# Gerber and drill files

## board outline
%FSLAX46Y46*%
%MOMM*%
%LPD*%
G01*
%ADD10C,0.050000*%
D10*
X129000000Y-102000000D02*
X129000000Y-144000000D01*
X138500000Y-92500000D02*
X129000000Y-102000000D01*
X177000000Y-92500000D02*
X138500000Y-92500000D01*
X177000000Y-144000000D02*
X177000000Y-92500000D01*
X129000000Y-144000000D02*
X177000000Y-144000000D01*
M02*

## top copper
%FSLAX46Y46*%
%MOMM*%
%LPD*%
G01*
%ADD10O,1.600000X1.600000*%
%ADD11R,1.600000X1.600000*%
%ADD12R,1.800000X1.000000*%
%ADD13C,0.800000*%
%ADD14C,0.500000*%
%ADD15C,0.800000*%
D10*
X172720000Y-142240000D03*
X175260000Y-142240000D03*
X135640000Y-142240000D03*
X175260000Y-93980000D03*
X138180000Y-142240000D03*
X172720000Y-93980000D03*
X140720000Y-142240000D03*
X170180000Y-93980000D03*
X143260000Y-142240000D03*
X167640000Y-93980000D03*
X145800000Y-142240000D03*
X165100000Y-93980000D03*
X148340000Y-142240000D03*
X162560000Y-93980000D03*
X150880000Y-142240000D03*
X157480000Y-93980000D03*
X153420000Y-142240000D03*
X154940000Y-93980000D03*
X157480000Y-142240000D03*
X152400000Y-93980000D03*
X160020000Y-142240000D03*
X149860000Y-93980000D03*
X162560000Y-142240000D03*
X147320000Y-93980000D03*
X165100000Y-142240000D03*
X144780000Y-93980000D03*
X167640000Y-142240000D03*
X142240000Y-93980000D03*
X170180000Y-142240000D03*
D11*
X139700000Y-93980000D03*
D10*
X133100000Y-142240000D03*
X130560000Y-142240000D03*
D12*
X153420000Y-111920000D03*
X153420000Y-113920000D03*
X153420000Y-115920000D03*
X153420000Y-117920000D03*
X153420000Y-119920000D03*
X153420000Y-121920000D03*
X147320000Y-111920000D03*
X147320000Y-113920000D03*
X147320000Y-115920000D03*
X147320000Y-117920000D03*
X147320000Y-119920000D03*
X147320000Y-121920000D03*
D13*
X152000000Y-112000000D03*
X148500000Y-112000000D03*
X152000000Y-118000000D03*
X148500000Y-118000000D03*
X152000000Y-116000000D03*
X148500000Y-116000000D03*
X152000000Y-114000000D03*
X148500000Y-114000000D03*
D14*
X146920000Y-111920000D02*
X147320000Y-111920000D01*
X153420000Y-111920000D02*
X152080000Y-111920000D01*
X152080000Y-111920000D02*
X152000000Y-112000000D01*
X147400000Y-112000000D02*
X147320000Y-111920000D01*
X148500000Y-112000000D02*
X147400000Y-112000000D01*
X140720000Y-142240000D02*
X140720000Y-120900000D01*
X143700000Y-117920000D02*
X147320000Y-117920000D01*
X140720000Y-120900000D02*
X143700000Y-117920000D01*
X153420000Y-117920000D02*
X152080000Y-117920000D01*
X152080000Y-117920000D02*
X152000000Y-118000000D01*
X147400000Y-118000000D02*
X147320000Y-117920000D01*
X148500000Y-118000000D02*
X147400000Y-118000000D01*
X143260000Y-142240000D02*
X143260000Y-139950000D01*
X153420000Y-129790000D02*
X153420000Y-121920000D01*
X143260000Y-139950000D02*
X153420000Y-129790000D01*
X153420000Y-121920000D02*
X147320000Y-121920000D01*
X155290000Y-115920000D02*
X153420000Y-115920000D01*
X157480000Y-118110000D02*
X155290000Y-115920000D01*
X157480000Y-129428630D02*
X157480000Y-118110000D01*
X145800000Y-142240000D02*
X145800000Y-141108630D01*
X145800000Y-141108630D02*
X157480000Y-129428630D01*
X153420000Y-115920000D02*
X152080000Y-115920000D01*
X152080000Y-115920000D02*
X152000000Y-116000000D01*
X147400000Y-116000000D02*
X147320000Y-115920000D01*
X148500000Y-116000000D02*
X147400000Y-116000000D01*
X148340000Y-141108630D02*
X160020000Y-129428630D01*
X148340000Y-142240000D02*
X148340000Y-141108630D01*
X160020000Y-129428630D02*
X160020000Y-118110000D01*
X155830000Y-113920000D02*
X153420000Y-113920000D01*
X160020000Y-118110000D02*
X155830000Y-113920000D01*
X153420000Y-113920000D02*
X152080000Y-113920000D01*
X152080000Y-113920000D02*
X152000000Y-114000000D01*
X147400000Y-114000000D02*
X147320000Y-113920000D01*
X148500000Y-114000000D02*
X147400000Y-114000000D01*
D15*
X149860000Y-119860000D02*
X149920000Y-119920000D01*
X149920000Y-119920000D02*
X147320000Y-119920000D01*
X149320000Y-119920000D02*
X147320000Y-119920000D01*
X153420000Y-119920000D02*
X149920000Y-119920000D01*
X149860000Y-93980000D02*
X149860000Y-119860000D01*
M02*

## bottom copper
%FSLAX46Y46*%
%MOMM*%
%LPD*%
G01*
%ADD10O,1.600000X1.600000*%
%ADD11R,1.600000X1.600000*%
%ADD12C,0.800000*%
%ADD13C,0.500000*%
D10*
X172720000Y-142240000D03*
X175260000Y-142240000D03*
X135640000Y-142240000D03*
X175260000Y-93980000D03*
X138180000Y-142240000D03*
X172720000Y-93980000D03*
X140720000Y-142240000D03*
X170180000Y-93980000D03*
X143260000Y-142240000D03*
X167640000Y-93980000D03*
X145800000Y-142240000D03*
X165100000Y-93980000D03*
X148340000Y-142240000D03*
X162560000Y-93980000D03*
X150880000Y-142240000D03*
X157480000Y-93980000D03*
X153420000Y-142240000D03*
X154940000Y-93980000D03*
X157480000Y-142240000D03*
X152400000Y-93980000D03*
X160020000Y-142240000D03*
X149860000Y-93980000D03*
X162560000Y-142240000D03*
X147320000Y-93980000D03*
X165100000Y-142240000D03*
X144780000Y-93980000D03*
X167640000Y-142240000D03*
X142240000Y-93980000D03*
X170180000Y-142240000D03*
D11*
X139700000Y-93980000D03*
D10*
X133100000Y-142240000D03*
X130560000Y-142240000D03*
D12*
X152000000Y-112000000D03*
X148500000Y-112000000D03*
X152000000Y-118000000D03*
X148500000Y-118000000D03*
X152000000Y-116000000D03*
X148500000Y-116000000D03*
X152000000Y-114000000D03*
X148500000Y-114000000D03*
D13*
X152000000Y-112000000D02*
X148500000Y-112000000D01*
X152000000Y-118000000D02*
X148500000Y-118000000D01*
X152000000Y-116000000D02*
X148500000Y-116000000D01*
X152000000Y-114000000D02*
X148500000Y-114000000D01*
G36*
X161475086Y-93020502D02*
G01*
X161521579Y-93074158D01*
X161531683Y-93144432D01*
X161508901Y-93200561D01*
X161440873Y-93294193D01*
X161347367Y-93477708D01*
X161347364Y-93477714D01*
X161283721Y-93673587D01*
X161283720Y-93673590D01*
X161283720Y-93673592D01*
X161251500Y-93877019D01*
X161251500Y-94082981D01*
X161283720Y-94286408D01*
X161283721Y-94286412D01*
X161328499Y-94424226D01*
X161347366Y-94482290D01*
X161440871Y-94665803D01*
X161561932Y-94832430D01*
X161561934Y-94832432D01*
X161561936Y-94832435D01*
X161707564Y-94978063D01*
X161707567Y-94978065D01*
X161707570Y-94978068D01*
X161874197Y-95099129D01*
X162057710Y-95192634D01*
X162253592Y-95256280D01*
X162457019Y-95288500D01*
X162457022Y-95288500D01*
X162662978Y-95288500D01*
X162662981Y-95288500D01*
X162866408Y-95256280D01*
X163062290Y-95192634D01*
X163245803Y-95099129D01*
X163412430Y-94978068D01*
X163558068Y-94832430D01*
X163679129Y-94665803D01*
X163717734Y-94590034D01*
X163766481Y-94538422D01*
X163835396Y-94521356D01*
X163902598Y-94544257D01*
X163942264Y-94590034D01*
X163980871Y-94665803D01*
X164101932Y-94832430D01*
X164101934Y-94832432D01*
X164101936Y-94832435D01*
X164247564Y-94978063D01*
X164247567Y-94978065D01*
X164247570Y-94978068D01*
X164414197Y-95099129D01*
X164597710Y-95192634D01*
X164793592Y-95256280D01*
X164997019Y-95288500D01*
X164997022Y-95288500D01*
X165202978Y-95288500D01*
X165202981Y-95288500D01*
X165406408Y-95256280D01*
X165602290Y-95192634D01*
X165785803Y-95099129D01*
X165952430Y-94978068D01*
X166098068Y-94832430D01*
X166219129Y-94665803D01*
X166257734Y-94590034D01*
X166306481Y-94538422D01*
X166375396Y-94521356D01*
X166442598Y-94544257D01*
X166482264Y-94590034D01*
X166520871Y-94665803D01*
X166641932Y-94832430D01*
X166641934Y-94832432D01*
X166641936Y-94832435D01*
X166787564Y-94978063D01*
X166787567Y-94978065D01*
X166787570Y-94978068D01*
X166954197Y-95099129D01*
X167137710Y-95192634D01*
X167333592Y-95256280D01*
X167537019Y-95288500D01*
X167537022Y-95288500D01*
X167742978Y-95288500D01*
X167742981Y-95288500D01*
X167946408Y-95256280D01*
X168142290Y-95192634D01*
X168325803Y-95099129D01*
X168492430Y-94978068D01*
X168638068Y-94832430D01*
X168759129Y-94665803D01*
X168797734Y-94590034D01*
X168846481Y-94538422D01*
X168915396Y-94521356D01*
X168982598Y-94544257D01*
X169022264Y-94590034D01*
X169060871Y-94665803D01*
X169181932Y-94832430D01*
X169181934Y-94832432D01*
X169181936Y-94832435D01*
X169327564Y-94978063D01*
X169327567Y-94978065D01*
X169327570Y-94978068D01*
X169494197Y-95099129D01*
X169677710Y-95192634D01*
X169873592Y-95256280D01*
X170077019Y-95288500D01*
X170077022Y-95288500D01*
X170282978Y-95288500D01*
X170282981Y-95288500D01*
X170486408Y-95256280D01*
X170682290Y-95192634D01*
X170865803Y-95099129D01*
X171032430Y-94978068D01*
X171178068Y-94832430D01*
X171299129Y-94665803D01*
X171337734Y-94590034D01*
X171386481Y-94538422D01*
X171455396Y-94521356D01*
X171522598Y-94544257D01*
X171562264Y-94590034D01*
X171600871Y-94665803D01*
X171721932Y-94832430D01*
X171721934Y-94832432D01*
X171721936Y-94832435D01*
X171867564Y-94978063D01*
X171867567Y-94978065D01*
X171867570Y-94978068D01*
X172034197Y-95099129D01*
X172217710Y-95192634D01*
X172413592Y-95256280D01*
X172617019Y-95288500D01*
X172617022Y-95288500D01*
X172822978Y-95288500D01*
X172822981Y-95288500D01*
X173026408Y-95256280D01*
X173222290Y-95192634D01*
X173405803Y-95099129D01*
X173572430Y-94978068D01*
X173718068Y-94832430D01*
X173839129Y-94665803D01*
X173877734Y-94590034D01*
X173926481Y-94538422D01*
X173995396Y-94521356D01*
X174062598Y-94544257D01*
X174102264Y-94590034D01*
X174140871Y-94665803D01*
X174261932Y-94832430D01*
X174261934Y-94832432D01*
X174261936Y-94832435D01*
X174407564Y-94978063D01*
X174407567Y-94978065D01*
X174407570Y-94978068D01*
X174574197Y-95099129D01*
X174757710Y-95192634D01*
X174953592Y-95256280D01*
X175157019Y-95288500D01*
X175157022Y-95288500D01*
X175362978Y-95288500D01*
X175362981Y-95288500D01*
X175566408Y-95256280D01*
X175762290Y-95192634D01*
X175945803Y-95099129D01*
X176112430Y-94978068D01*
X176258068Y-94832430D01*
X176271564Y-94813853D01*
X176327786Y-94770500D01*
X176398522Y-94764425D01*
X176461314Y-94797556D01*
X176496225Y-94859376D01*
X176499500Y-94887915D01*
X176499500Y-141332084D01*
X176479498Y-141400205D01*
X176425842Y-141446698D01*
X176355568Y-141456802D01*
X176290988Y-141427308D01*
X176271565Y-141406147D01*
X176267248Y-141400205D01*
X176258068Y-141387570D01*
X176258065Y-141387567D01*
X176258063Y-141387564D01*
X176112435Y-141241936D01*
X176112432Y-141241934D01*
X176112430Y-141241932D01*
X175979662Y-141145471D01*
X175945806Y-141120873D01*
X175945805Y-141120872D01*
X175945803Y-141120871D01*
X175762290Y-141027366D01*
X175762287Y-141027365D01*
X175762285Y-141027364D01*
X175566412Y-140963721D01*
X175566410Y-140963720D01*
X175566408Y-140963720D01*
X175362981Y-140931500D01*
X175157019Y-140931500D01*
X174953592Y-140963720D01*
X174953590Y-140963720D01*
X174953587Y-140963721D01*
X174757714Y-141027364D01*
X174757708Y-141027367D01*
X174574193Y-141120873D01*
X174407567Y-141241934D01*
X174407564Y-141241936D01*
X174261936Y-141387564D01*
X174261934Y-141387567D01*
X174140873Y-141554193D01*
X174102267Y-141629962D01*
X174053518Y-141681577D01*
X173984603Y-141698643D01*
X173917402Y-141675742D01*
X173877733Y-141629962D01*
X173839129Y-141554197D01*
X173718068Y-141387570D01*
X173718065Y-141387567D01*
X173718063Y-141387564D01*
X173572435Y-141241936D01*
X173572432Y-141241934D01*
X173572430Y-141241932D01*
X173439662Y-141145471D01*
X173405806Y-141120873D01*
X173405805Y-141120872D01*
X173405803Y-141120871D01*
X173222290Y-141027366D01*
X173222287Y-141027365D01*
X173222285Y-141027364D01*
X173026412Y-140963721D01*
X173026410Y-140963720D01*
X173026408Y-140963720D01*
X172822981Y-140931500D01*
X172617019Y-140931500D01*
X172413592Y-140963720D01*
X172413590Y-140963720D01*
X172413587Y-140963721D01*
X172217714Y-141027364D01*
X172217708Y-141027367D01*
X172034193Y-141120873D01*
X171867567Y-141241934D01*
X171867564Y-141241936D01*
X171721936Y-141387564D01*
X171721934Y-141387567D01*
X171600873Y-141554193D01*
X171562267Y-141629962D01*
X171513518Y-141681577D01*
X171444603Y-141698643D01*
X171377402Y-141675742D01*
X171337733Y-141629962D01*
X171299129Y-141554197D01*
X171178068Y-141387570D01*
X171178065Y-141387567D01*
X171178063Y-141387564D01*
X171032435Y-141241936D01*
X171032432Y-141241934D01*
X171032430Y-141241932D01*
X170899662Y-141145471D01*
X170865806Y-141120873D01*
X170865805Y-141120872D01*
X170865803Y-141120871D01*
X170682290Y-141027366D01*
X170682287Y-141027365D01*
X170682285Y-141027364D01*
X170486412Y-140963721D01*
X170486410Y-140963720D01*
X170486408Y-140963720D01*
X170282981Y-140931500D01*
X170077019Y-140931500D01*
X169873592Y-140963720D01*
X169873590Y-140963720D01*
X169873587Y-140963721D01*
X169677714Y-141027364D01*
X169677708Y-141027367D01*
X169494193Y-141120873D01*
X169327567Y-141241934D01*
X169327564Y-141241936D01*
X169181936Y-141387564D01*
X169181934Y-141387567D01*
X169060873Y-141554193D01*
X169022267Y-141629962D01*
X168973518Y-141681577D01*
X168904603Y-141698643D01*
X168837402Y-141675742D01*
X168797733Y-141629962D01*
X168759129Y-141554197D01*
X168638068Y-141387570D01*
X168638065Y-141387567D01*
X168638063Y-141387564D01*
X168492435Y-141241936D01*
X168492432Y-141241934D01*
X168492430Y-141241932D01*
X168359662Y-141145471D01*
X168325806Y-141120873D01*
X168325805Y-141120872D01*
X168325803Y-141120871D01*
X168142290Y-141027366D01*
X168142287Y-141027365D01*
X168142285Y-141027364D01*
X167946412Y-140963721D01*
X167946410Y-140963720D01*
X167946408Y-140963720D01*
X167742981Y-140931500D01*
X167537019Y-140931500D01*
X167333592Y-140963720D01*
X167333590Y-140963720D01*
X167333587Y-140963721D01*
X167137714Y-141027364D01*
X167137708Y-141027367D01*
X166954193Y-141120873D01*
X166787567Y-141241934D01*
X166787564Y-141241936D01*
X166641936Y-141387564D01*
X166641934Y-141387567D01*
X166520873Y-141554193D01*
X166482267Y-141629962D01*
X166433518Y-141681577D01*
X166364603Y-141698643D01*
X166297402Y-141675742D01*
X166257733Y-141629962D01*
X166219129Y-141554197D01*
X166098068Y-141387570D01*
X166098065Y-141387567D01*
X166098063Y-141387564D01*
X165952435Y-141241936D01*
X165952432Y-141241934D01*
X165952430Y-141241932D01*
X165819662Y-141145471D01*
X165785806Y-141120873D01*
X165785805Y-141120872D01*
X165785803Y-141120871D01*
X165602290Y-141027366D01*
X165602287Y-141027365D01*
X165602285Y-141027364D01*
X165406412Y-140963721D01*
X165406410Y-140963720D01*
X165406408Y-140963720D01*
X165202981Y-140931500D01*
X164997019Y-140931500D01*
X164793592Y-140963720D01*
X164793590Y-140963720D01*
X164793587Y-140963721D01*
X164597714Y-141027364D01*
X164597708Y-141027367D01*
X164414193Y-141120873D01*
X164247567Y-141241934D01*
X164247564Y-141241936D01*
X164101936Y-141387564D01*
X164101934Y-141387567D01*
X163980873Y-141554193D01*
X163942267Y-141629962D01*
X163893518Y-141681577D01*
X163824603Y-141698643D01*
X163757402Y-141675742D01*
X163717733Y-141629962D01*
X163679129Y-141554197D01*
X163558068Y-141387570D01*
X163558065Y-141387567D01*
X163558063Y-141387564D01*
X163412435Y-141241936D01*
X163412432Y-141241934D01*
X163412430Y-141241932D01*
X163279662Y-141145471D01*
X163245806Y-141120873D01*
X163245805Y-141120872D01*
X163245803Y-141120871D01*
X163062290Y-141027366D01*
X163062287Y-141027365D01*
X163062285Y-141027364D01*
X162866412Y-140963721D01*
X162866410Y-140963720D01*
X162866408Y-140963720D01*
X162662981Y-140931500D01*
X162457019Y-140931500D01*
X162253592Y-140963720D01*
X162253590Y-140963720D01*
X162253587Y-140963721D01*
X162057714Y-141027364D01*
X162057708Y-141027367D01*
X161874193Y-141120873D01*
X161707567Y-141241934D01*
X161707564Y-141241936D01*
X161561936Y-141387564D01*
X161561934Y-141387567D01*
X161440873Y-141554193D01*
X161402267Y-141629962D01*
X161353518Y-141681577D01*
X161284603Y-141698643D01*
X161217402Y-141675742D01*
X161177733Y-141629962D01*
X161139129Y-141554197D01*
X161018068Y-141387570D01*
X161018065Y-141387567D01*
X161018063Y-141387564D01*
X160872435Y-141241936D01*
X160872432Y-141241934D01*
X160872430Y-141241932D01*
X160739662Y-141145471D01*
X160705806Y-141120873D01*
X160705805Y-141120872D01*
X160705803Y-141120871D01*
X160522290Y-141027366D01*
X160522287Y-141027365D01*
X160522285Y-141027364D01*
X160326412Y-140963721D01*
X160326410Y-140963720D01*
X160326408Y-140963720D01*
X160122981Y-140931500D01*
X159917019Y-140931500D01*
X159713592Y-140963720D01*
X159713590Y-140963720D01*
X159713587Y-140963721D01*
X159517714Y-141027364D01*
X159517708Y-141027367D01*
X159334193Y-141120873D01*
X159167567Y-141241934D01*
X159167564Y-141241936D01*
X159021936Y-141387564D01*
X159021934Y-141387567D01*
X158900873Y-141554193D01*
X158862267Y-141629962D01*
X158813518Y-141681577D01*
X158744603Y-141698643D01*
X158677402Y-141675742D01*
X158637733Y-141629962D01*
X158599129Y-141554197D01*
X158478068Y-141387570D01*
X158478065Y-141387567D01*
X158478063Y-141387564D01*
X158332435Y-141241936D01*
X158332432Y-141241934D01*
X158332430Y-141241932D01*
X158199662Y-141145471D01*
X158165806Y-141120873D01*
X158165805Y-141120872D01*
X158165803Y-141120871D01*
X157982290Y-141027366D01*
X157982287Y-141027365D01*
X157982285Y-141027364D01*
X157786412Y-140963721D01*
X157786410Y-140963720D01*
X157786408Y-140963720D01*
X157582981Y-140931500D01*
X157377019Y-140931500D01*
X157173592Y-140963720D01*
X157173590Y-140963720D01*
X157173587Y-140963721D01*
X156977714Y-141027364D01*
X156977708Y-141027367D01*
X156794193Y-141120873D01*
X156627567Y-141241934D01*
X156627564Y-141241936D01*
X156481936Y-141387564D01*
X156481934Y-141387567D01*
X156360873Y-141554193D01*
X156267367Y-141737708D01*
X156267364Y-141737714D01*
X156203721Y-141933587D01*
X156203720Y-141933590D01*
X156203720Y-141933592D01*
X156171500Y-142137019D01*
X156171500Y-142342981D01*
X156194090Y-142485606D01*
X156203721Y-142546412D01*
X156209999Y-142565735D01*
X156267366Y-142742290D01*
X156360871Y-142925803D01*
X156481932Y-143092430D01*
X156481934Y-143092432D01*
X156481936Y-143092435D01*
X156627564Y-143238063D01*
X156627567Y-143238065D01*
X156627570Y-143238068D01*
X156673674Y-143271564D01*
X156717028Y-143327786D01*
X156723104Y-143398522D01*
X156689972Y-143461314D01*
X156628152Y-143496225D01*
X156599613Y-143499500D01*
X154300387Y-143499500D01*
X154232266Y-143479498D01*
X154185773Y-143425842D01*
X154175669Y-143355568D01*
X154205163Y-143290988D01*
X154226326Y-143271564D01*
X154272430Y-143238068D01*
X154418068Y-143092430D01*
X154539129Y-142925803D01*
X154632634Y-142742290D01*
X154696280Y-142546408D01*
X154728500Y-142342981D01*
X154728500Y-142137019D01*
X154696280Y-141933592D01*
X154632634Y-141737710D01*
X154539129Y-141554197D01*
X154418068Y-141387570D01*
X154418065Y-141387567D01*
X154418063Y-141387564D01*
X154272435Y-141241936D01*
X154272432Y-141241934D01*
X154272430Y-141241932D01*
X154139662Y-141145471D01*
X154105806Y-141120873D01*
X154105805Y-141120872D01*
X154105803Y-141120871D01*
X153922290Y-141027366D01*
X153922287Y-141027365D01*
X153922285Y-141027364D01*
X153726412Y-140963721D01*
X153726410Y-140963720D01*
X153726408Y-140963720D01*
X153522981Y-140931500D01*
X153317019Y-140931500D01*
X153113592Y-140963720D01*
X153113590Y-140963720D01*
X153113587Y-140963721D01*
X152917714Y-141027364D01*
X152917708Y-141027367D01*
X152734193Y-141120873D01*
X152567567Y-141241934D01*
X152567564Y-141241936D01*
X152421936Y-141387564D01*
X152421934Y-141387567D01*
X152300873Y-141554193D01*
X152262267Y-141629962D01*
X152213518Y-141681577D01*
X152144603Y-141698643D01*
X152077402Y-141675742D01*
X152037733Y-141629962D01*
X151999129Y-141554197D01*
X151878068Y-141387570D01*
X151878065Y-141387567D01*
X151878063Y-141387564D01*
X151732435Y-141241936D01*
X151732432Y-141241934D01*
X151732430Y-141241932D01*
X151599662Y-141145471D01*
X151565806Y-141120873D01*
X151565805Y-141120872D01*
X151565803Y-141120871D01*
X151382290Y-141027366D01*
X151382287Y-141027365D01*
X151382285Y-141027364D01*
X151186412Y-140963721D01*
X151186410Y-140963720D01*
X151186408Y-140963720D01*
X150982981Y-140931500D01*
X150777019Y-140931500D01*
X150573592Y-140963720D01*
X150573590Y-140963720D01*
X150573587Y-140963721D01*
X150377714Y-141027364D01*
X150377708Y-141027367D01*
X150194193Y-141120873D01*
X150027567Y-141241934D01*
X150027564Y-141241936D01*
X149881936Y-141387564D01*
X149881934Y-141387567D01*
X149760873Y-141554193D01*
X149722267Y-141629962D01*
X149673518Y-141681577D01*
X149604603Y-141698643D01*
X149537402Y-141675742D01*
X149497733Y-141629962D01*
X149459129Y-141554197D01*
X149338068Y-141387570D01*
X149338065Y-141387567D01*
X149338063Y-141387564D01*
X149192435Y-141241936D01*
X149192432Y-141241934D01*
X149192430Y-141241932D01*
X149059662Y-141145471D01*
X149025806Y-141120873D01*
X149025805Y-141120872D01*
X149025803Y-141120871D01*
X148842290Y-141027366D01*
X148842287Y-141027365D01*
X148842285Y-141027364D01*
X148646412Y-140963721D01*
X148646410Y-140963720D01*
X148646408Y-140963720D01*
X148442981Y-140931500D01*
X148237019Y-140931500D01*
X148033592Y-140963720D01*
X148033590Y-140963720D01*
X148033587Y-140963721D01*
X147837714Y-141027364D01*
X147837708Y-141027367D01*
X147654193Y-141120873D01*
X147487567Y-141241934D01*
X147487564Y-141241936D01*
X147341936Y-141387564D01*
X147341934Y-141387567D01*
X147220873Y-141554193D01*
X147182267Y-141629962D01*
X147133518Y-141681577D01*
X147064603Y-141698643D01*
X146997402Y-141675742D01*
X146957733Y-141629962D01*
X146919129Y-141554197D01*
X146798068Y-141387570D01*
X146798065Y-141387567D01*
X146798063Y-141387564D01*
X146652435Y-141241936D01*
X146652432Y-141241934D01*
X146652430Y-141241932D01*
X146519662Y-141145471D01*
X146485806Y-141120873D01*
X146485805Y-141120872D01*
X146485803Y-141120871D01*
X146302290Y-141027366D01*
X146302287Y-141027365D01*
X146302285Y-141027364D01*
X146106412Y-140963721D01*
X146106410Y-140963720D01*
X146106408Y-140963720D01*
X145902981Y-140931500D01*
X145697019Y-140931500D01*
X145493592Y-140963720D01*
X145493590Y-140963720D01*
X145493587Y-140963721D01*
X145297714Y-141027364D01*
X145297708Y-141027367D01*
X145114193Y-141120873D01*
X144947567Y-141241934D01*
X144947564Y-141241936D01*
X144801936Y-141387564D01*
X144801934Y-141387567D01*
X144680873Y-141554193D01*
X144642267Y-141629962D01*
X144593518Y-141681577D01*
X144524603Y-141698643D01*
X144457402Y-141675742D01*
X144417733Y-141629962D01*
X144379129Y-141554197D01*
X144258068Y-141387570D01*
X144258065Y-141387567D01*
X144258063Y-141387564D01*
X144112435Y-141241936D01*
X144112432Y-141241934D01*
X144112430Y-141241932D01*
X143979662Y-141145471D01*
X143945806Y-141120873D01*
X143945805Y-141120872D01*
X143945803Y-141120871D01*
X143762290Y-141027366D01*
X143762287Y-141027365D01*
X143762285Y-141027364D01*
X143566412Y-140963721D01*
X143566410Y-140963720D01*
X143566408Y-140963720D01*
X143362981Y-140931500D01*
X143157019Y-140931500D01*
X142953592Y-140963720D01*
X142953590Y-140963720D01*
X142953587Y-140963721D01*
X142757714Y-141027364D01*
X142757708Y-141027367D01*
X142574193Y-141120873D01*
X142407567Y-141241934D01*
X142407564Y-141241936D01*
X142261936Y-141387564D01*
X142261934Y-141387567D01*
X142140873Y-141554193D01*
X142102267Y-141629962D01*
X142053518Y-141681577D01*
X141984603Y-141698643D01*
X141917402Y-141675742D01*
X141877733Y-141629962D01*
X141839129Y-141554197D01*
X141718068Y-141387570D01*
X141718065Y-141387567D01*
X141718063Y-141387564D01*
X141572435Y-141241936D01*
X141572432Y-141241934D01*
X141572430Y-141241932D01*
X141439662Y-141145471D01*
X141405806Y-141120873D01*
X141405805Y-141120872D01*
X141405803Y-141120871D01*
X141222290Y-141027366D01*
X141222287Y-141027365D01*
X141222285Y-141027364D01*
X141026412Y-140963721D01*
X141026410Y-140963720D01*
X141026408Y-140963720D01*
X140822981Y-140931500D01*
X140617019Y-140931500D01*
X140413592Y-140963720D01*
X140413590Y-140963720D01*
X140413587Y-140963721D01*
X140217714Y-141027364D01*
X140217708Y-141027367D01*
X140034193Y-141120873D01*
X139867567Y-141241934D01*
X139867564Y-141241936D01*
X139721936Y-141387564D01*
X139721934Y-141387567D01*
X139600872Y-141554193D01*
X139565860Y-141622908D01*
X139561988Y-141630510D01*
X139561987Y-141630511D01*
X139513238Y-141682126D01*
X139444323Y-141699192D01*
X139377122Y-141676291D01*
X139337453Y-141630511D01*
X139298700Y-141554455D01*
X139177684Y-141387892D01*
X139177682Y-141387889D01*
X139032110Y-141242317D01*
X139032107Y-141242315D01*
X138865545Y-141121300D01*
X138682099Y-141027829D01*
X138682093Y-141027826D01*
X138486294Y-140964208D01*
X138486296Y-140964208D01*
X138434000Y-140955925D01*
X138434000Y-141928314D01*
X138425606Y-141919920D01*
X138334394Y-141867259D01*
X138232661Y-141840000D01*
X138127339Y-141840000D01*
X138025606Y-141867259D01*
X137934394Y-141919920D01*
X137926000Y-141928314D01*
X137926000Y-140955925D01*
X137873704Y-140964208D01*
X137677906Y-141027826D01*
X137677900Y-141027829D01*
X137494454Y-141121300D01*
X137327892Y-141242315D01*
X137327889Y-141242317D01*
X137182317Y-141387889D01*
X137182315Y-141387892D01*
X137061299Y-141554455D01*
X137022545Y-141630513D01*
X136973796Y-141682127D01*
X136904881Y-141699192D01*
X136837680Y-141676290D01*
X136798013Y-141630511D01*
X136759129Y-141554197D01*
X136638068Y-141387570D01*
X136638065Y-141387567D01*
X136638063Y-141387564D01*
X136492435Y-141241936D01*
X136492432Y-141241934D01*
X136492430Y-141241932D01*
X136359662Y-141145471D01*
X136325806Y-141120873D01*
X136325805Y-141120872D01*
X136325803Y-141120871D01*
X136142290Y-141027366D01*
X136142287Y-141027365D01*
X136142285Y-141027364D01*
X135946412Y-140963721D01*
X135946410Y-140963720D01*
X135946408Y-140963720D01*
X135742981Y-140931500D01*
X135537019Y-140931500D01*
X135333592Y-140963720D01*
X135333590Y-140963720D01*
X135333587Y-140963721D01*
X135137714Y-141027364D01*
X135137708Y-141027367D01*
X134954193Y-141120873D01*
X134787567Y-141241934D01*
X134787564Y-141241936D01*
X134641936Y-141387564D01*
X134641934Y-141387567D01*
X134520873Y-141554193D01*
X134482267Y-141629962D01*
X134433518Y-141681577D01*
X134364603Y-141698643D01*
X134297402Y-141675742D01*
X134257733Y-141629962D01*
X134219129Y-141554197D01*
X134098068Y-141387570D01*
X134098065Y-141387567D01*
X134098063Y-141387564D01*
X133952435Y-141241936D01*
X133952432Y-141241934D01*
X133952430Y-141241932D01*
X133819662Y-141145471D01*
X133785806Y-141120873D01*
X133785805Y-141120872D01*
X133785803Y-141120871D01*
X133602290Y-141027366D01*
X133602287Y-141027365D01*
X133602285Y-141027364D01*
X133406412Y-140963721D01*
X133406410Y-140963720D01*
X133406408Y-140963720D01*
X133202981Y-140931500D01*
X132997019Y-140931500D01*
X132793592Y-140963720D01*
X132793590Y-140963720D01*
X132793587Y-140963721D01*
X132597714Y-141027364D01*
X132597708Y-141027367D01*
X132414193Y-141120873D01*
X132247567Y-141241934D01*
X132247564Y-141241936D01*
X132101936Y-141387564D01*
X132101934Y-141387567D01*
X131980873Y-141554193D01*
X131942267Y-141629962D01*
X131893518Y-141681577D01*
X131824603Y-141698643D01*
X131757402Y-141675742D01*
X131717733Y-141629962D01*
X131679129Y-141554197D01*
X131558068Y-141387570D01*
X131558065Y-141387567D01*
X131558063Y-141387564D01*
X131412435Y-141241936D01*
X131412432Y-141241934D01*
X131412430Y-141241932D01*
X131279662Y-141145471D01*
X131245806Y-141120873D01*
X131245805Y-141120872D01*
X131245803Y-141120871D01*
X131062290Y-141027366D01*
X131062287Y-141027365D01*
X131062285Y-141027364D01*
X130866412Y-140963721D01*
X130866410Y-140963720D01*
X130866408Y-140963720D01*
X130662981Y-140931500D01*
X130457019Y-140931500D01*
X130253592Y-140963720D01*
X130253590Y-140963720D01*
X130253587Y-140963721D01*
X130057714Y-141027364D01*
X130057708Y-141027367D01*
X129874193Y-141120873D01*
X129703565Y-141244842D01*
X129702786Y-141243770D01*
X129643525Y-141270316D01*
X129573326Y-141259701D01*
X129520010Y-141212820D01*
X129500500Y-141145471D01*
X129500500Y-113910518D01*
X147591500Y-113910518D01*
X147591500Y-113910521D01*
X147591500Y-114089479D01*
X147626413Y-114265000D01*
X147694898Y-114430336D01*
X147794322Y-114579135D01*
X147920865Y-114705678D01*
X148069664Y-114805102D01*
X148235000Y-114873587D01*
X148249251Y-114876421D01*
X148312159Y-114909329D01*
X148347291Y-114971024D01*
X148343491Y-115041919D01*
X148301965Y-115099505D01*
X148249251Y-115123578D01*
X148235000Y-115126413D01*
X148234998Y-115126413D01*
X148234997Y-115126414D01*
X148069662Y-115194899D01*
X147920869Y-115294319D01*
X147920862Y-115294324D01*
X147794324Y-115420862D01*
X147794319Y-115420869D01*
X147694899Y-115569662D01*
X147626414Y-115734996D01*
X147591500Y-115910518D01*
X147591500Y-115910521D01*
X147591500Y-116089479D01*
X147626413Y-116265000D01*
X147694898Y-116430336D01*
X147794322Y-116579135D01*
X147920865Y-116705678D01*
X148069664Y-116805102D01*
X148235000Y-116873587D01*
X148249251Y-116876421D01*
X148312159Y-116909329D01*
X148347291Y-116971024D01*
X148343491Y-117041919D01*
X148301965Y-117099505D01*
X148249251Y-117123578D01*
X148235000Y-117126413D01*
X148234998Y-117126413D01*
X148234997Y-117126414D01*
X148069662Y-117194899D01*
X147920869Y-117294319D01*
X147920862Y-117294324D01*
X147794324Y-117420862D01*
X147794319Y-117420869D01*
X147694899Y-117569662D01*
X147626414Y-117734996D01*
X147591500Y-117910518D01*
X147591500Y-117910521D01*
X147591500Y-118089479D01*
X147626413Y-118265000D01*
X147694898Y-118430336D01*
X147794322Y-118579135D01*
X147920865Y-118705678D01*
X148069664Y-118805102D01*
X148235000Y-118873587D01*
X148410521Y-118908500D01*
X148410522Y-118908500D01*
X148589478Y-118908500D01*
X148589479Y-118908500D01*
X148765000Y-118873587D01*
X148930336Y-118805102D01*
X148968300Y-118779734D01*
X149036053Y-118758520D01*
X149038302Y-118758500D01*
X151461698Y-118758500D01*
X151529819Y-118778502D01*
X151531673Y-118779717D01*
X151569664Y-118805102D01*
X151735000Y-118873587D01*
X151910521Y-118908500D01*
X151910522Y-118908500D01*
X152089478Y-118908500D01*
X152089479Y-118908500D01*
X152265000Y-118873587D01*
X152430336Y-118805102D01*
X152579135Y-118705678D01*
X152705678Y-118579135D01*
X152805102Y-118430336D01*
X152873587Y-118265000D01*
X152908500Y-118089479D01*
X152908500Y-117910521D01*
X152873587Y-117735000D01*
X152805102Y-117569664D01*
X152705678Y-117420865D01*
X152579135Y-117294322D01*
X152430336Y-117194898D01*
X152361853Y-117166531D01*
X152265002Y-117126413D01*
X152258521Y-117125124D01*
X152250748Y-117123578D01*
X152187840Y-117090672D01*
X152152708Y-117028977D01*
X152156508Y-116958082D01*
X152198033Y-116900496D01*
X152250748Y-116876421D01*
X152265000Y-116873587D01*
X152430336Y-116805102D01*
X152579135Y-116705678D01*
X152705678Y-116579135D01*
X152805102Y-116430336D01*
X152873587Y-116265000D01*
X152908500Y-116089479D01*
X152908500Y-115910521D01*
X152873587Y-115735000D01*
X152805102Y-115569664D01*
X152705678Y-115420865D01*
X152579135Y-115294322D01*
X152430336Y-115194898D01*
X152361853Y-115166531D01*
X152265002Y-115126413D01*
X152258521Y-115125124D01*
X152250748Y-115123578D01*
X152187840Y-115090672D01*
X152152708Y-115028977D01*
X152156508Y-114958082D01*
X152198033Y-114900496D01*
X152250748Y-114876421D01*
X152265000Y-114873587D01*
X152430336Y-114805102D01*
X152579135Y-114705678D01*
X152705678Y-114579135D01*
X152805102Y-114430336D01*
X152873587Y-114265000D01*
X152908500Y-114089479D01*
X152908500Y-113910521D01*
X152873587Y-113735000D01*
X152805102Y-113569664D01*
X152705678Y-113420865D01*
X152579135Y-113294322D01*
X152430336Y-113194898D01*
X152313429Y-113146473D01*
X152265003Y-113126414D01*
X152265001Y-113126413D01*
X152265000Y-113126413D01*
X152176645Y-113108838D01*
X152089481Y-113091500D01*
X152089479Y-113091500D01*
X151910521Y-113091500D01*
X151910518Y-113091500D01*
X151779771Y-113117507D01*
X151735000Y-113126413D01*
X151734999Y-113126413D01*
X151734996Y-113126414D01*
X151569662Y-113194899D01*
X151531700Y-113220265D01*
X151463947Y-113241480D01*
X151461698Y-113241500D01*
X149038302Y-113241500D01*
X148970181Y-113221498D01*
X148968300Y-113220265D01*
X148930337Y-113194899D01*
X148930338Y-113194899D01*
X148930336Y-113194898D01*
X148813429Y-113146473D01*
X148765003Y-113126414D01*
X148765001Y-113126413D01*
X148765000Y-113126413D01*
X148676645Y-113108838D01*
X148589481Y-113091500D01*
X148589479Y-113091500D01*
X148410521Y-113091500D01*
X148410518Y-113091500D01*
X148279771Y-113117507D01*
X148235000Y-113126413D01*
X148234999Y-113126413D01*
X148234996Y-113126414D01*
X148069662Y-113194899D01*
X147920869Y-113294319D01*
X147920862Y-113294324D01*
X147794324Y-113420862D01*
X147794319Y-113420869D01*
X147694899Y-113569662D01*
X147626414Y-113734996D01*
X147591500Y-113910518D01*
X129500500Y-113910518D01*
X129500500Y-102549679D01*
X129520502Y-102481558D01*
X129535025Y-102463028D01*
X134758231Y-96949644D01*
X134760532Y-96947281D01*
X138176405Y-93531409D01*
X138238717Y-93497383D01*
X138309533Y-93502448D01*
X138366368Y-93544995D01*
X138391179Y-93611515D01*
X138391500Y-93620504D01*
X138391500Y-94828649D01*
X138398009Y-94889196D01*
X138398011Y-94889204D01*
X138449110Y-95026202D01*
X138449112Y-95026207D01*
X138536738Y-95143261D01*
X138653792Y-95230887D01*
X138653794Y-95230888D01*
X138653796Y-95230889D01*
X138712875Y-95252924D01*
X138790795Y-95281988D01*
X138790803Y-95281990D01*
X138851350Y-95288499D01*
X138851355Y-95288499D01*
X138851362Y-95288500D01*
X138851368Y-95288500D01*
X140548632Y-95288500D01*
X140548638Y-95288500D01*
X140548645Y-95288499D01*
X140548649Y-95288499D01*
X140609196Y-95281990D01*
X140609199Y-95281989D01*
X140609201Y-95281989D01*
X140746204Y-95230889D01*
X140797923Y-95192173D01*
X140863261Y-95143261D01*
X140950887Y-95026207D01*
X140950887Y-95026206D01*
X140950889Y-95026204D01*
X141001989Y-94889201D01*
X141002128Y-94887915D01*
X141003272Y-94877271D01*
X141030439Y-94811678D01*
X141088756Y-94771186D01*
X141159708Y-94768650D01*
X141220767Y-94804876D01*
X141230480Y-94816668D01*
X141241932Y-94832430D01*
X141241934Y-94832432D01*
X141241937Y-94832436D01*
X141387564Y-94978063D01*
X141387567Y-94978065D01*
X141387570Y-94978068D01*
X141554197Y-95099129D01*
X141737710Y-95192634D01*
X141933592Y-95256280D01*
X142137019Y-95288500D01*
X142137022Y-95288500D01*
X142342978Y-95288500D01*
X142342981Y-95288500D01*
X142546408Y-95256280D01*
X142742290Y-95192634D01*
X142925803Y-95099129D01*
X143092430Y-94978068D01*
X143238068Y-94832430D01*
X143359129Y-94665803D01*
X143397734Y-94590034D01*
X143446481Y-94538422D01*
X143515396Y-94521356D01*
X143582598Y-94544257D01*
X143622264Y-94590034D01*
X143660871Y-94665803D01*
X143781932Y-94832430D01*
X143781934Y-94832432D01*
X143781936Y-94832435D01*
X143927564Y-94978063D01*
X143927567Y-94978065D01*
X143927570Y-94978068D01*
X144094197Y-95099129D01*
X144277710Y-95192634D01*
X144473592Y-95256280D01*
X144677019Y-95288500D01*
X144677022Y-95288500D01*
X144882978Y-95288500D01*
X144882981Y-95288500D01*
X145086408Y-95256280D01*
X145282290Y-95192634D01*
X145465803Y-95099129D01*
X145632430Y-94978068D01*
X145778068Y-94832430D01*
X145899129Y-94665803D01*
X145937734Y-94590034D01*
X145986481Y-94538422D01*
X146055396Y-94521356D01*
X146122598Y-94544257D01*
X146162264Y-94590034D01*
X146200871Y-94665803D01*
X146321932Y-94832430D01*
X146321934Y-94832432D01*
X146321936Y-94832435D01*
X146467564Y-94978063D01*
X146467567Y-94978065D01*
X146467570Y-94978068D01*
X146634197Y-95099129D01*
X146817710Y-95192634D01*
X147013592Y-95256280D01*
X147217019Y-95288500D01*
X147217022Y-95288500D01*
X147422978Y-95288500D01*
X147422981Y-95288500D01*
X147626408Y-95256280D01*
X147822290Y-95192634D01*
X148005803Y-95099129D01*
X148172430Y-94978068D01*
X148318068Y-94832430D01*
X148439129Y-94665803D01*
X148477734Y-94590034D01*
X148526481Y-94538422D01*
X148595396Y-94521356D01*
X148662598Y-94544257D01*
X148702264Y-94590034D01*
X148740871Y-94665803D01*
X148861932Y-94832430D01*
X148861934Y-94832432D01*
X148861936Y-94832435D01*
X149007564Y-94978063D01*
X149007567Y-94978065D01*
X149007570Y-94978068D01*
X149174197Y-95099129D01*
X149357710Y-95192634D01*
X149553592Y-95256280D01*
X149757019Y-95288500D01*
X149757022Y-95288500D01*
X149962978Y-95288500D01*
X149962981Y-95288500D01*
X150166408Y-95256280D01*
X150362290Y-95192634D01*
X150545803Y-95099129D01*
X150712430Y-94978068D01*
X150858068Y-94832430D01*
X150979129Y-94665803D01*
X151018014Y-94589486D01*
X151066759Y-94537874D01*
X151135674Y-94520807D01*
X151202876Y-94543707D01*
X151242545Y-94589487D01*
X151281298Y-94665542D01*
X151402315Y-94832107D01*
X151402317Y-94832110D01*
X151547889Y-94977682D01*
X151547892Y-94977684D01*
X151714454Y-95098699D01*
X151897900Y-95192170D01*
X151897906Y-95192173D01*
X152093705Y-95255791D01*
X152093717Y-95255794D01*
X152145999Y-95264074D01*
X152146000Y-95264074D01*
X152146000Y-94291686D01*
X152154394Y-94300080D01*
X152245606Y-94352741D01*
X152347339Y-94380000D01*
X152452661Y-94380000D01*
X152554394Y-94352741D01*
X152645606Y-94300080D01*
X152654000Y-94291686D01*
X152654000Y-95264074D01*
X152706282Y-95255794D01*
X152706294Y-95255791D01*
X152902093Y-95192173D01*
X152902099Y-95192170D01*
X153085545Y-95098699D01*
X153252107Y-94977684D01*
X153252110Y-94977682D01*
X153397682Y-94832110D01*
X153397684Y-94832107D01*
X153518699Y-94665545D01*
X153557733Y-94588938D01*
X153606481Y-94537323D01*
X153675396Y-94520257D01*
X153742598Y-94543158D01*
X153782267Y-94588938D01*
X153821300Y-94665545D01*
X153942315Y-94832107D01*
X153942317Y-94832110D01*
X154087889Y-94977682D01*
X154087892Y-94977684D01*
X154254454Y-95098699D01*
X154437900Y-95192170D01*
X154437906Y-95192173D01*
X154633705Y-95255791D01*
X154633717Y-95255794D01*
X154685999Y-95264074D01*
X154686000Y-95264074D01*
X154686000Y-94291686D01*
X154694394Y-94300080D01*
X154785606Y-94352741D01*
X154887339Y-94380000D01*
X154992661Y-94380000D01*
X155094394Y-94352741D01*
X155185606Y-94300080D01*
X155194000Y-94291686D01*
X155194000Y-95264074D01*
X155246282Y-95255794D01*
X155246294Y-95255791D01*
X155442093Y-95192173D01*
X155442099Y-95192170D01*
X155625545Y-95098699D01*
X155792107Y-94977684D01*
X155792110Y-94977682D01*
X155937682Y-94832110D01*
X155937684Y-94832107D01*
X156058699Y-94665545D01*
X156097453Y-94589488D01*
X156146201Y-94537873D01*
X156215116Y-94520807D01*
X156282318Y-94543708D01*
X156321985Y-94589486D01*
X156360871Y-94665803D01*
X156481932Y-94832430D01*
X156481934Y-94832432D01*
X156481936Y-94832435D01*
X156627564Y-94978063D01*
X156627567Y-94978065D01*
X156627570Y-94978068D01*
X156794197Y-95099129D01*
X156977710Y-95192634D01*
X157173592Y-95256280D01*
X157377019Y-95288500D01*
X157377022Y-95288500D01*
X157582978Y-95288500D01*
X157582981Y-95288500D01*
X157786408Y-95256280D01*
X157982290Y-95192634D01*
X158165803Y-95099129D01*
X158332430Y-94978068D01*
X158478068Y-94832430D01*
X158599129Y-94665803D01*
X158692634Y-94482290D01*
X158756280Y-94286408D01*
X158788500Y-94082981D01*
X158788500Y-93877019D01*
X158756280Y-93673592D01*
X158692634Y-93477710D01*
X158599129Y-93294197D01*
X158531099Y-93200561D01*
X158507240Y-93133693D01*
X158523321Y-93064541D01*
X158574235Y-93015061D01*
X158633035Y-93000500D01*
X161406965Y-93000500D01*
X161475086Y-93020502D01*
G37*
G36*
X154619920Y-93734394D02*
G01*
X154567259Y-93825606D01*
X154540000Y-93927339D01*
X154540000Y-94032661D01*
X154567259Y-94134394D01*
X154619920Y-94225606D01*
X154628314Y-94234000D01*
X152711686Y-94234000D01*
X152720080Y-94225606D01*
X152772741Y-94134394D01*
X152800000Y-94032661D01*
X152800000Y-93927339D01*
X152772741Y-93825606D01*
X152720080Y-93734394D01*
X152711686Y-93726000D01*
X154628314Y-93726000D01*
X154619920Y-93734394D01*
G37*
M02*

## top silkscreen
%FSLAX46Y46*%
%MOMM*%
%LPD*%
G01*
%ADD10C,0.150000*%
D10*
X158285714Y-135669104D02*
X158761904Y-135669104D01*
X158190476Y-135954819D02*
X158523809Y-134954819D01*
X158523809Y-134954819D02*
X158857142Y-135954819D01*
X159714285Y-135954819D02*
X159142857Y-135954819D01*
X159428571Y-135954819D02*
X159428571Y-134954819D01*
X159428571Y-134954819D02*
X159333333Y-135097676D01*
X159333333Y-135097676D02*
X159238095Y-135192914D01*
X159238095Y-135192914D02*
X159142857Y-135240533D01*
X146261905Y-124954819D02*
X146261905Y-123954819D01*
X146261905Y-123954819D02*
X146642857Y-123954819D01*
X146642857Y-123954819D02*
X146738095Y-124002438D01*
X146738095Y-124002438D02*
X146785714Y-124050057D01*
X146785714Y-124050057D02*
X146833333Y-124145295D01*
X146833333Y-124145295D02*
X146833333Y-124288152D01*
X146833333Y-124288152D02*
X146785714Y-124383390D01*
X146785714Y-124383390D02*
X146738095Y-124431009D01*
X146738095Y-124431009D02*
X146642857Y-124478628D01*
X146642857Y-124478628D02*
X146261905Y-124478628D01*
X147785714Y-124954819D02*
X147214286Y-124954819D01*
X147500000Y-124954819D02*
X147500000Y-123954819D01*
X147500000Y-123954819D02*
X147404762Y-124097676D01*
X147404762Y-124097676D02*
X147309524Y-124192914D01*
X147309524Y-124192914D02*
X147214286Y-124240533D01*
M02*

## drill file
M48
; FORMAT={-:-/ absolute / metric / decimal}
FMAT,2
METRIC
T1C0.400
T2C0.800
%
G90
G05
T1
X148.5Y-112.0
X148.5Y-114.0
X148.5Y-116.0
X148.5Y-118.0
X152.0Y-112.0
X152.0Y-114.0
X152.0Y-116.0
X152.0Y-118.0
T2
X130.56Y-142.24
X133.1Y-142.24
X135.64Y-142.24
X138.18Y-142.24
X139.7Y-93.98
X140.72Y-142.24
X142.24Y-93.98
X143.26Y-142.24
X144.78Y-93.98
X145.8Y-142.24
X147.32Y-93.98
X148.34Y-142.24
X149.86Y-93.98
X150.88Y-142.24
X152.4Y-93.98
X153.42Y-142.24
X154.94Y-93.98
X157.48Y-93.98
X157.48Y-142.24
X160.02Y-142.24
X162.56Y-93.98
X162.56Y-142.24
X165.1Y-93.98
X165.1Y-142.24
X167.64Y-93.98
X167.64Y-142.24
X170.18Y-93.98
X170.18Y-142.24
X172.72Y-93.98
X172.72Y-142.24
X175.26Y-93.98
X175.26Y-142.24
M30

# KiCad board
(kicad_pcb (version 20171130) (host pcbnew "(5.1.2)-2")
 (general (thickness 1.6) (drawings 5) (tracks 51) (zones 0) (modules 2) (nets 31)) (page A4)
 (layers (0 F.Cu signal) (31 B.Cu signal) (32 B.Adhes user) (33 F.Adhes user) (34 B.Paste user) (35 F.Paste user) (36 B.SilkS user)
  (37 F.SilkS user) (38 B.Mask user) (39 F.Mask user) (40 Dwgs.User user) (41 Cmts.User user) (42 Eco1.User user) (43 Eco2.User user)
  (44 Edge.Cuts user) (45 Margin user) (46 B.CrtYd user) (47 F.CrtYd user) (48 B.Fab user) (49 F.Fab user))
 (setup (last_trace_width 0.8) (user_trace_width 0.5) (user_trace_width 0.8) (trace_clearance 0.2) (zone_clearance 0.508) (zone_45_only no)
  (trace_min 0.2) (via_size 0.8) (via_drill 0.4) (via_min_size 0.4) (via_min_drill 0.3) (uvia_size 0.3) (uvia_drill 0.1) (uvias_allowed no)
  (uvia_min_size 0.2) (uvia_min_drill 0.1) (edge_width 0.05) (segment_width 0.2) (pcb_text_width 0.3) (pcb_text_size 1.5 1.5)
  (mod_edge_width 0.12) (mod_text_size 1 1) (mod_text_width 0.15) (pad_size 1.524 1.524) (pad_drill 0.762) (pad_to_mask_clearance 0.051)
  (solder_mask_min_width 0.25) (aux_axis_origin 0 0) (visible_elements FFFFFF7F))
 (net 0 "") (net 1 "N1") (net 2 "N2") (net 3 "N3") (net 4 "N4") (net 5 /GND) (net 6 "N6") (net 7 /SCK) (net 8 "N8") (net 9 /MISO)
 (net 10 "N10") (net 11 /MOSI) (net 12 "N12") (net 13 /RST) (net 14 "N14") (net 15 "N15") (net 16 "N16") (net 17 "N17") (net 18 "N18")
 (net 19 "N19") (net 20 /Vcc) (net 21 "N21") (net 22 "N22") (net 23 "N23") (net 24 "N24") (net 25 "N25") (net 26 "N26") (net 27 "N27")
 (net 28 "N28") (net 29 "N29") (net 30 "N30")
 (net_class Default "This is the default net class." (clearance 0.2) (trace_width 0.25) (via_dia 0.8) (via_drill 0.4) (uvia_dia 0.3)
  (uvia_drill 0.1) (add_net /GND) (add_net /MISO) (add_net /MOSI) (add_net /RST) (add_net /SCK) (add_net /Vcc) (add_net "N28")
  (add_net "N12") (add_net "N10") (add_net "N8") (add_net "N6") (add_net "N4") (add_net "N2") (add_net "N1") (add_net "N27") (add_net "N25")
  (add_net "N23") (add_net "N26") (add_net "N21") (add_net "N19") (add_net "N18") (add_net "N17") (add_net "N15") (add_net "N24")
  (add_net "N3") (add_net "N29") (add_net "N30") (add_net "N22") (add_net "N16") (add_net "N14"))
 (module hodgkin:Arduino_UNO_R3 (layer F.Cu) (at 139.7 93.98)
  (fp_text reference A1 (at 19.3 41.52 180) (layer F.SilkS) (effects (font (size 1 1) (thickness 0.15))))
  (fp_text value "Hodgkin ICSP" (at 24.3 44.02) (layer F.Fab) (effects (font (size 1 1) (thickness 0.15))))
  (pad 16 thru_hole oval (at 33.02 48.26 90) (size 1.6 1.6) (drill 0.8) (layers *.Cu *.Mask) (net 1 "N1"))
  (pad 15 thru_hole oval (at 35.56 48.26 90) (size 1.6 1.6) (drill 0.8) (layers *.Cu *.Mask) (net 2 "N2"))
  (pad 30 thru_hole oval (at -4.06 48.26 90) (size 1.6 1.6) (drill 0.8) (layers *.Cu *.Mask) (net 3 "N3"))
  (pad 14 thru_hole oval (at 35.56 0 90) (size 1.6 1.6) (drill 0.8) (layers *.Cu *.Mask) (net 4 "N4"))
  (pad 29 thru_hole oval (at -1.52 48.26 90) (size 1.6 1.6) (drill 0.8) (layers *.Cu *.Mask) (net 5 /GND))
  (pad 13 thru_hole oval (at 33.02 0 90) (size 1.6 1.6) (drill 0.8) (layers *.Cu *.Mask) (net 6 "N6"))
  (pad 28 thru_hole oval (at 1.02 48.26 90) (size 1.6 1.6) (drill 0.8) (layers *.Cu *.Mask) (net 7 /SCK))
  (pad 12 thru_hole oval (at 30.48 0 90) (size 1.6 1.6) (drill 0.8) (layers *.Cu *.Mask) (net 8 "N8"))
  (pad 27 thru_hole oval (at 3.56 48.26 90) (size 1.6 1.6) (drill 0.8) (layers *.Cu *.Mask) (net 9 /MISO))
  (pad 11 thru_hole oval (at 27.94 0 90) (size 1.6 1.6) (drill 0.8) (layers *.Cu *.Mask) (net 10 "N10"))
  (pad 26 thru_hole oval (at 6.1 48.26 90) (size 1.6 1.6) (drill 0.8) (layers *.Cu *.Mask) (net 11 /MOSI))
  (pad 10 thru_hole oval (at 25.4 0 90) (size 1.6 1.6) (drill 0.8) (layers *.Cu *.Mask) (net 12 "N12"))
  (pad 25 thru_hole oval (at 8.64 48.26 90) (size 1.6 1.6) (drill 0.8) (layers *.Cu *.Mask) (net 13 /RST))
  (pad 9 thru_hole oval (at 22.86 0 90) (size 1.6 1.6) (drill 0.8) (layers *.Cu *.Mask) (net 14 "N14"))
  (pad 24 thru_hole oval (at 11.18 48.26 90) (size 1.6 1.6) (drill 0.8) (layers *.Cu *.Mask) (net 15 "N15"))
  (pad 8 thru_hole oval (at 17.78 0 90) (size 1.6 1.6) (drill 0.8) (layers *.Cu *.Mask) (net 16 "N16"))
  (pad 23 thru_hole oval (at 13.72 48.26 90) (size 1.6 1.6) (drill 0.8) (layers *.Cu *.Mask) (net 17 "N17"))
  (pad 7 thru_hole oval (at 15.24 0 90) (size 1.6 1.6) (drill 0.8) (layers *.Cu *.Mask) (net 5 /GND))
  (pad 22 thru_hole oval (at 17.78 48.26 90) (size 1.6 1.6) (drill 0.8) (layers *.Cu *.Mask) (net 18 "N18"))
  (pad 6 thru_hole oval (at 12.7 0 90) (size 1.6 1.6) (drill 0.8) (layers *.Cu *.Mask) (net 5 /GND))
  (pad 21 thru_hole oval (at 20.32 48.26 90) (size 1.6 1.6) (drill 0.8) (layers *.Cu *.Mask) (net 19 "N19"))
  (pad 5 thru_hole oval (at 10.16 0 90) (size 1.6 1.6) (drill 0.8) (layers *.Cu *.Mask) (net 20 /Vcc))
  (pad 20 thru_hole oval (at 22.86 48.26 90) (size 1.6 1.6) (drill 0.8) (layers *.Cu *.Mask) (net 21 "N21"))
  (pad 4 thru_hole oval (at 7.62 0 90) (size 1.6 1.6) (drill 0.8) (layers *.Cu *.Mask) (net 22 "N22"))
  (pad 19 thru_hole oval (at 25.4 48.26 90) (size 1.6 1.6) (drill 0.8) (layers *.Cu *.Mask) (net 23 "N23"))
  (pad 3 thru_hole oval (at 5.08 0 90) (size 1.6 1.6) (drill 0.8) (layers *.Cu *.Mask) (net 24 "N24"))
  (pad 18 thru_hole oval (at 27.94 48.26 90) (size 1.6 1.6) (drill 0.8) (layers *.Cu *.Mask) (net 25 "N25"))
  (pad 2 thru_hole oval (at 2.54 0 90) (size 1.6 1.6) (drill 0.8) (layers *.Cu *.Mask) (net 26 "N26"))
  (pad 17 thru_hole oval (at 30.48 48.26 90) (size 1.6 1.6) (drill 0.8) (layers *.Cu *.Mask) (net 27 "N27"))
  (pad 1 thru_hole rect (at 0 0 90) (size 1.6 1.6) (drill 0.8) (layers *.Cu *.Mask) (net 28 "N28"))
  (pad 31 thru_hole oval (at -6.6 48.26 90) (size 1.6 1.6) (drill 0.8) (layers *.Cu *.Mask) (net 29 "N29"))
  (pad 32 thru_hole oval (at -9.14 48.26 90) (size 1.6 1.6) (drill 0.8) (layers *.Cu *.Mask) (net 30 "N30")))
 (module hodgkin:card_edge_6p (layer F.Cu) (at 147.32 121.92 90)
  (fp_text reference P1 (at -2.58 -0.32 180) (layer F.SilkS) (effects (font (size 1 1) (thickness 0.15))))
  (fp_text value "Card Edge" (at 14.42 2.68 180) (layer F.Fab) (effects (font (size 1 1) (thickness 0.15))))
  (pad 6 smd rect (at 10 6.1 90) (size 1 1.8) (layers F.Cu F.Paste F.Mask) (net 5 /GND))
  (pad 5 smd rect (at 8 6.1 90) (size 1 1.8) (layers F.Cu F.Paste F.Mask) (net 13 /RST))
  (pad 4 smd rect (at 6 6.1 90) (size 1 1.8) (layers F.Cu F.Paste F.Mask) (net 11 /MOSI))
  (pad 3 smd rect (at 4 6.1 90) (size 1 1.8) (layers F.Cu F.Paste F.Mask) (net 7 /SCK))
  (pad 2 smd rect (at 2 6.1 90) (size 1 1.8) (layers F.Cu F.Paste F.Mask) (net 20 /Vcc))
  (pad 1 smd rect (at 0 6.1 90) (size 1 1.8) (layers F.Cu F.Paste F.Mask) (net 9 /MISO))
  (pad 6 smd rect (at 10 0 90) (size 1 1.8) (layers F.Cu F.Paste F.Mask) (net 5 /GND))
  (pad 5 smd rect (at 8 0 90) (size 1 1.8) (layers F.Cu F.Paste F.Mask) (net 13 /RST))
  (pad 4 smd rect (at 6 0 90) (size 1 1.8) (layers F.Cu F.Paste F.Mask) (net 11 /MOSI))
  (pad 3 smd rect (at 4 0 90) (size 1 1.8) (layers F.Cu F.Paste F.Mask) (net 7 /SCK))
  (pad 2 smd rect (at 2 0 90) (size 1 1.8) (layers F.Cu F.Paste F.Mask) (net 20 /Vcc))
  (pad 1 smd rect (at 0 0 90) (size 1 1.8) (layers F.Cu F.Paste F.Mask) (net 9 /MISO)))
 (gr_line (start 129 102) (end 129 144) (layer Edge.Cuts) (width 0.05))
 (gr_line (start 138.5 92.5) (end 129 102) (layer Edge.Cuts) (width 0.05))
 (gr_line (start 177 92.5) (end 138.5 92.5) (layer Edge.Cuts) (width 0.05))
 (gr_line (start 177 144) (end 177 92.5) (layer Edge.Cuts) (width 0.05))
 (gr_line (start 129 144) (end 177 144) (layer Edge.Cuts) (width 0.05))
 (segment (start 146.92 111.92) (end 147.32 111.92) (width 0.5) (layer F.Cu) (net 5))
 (via (at 152 112) (size 0.8) (drill 0.4) (layers F.Cu B.Cu) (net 5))
 (segment (start 153.42 111.92) (end 152.08 111.92) (width 0.5) (layer F.Cu) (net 5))
 (segment (start 152.08 111.92) (end 152 112) (width 0.5) (layer F.Cu) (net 5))
 (via (at 148.5 112) (size 0.8) (drill 0.4) (layers F.Cu B.Cu) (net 5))
 (segment (start 152 112) (end 148.5 112) (width 0.5) (layer B.Cu) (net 5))
 (segment (start 147.4 112) (end 147.32 111.92) (width 0.5) (layer F.Cu) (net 5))
 (segment (start 148.5 112) (end 147.4 112) (width 0.5) (layer F.Cu) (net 5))
 (segment (start 140.72 142.24) (end 140.72 120.9) (width 0.5) (layer F.Cu) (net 7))
 (segment (start 143.7 117.92) (end 147.32 117.92) (width 0.5) (layer F.Cu) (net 7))
 (segment (start 140.72 120.9) (end 143.7 117.92) (width 0.5) (layer F.Cu) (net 7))
 (via (at 152 118) (size 0.8) (drill 0.4) (layers F.Cu B.Cu) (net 7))
 (segment (start 153.42 117.92) (end 152.08 117.92) (width 0.5) (layer F.Cu) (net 7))
 (segment (start 152.08 117.92) (end 152 118) (width 0.5) (layer F.Cu) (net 7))
 (segment (start 152 118) (end 148.5 118) (width 0.5) (layer B.Cu) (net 7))
 (via (at 148.5 118) (size 0.8) (drill 0.4) (layers F.Cu B.Cu) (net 7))
 (segment (start 147.4 118) (end 147.32 117.92) (width 0.5) (layer F.Cu) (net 7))
 (segment (start 148.5 118) (end 147.4 118) (width 0.5) (layer F.Cu) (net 7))
 (segment (start 143.26 142.24) (end 143.26 139.95) (width 0.5) (layer F.Cu) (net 9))
 (segment (start 153.42 129.79) (end 153.42 121.92) (width 0.5) (layer F.Cu) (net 9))
 (segment (start 143.26 139.95) (end 153.42 129.79) (width 0.5) (layer F.Cu) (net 9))
 (segment (start 153.42 121.92) (end 147.32 121.92) (width 0.5) (layer F.Cu) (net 9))
 (segment (start 155.29 115.92) (end 153.42 115.92) (width 0.5) (layer F.Cu) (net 11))
 (segment (start 157.48 118.11) (end 155.29 115.92) (width 0.5) (layer F.Cu) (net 11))
 (segment (start 157.48 129.42863) (end 157.48 118.11) (width 0.5) (layer F.Cu) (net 11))
 (segment (start 145.8 142.24) (end 145.8 141.10863) (width 0.5) (layer F.Cu) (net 11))
 (segment (start 145.8 141.10863) (end 157.48 129.42863) (width 0.5) (layer F.Cu) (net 11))
 (via (at 152 116) (size 0.8) (drill 0.4) (layers F.Cu B.Cu) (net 11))
 (segment (start 153.42 115.92) (end 152.08 115.92) (width 0.5) (layer F.Cu) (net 11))
 (segment (start 152.08 115.92) (end 152 116) (width 0.5) (layer F.Cu) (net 11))
 (via (at 148.5 116) (size 0.8) (drill 0.4) (layers F.Cu B.Cu) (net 11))
 (segment (start 152 116) (end 148.5 116) (width 0.5) (layer B.Cu) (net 11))
 (segment (start 147.4 116) (end 147.32 115.92) (width 0.5) (layer F.Cu) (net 11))
 (segment (start 148.5 116) (end 147.4 116) (width 0.5) (layer F.Cu) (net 11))
 (segment (start 148.34 141.10863) (end 160.02 129.42863) (width 0.5) (layer F.Cu) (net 13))
 (segment (start 148.34 142.24) (end 148.34 141.10863) (width 0.5) (layer F.Cu) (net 13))
 (segment (start 160.02 129.42863) (end 160.02 118.11) (width 0.5) (layer F.Cu) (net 13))
 (segment (start 155.83 113.92) (end 153.42 113.92) (width 0.5) (layer F.Cu) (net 13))
 (segment (start 160.02 118.11) (end 155.83 113.92) (width 0.5) (layer F.Cu) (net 13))
 (via (at 152 114) (size 0.8) (drill 0.4) (layers F.Cu B.Cu) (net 13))
 (segment (start 153.42 113.92) (end 152.08 113.92) (width 0.5) (layer F.Cu) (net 13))
 (segment (start 152.08 113.92) (end 152 114) (width 0.5) (layer F.Cu) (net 13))
 (via (at 148.5 114) (size 0.8) (drill 0.4) (layers F.Cu B.Cu) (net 13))
 (segment (start 152 114) (end 148.5 114) (width 0.5) (layer B.Cu) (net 13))
 (segment (start 147.4 114) (end 147.32 113.92) (width 0.5) (layer F.Cu) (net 13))
 (segment (start 148.5 114) (end 147.4 114) (width 0.5) (layer F.Cu) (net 13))
 (segment (start 149.86 119.86) (end 149.92 119.92) (width 0.8) (layer F.Cu) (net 20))
 (segment (start 149.92 119.92) (end 147.32 119.92) (width 0.8) (layer F.Cu) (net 20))
 (segment (start 149.32 119.92) (end 147.32 119.92) (width 0.8) (layer F.Cu) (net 20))
 (segment (start 153.42 119.92) (end 149.92 119.92) (width 0.8) (layer F.Cu) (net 20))
 (segment (start 149.86 93.98) (end 149.86 119.86) (width 0.8) (layer F.Cu) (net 20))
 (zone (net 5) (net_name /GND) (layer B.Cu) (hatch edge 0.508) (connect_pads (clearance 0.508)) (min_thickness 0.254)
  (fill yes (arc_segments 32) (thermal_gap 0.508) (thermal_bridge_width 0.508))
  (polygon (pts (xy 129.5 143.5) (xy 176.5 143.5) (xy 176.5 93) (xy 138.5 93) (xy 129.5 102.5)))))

